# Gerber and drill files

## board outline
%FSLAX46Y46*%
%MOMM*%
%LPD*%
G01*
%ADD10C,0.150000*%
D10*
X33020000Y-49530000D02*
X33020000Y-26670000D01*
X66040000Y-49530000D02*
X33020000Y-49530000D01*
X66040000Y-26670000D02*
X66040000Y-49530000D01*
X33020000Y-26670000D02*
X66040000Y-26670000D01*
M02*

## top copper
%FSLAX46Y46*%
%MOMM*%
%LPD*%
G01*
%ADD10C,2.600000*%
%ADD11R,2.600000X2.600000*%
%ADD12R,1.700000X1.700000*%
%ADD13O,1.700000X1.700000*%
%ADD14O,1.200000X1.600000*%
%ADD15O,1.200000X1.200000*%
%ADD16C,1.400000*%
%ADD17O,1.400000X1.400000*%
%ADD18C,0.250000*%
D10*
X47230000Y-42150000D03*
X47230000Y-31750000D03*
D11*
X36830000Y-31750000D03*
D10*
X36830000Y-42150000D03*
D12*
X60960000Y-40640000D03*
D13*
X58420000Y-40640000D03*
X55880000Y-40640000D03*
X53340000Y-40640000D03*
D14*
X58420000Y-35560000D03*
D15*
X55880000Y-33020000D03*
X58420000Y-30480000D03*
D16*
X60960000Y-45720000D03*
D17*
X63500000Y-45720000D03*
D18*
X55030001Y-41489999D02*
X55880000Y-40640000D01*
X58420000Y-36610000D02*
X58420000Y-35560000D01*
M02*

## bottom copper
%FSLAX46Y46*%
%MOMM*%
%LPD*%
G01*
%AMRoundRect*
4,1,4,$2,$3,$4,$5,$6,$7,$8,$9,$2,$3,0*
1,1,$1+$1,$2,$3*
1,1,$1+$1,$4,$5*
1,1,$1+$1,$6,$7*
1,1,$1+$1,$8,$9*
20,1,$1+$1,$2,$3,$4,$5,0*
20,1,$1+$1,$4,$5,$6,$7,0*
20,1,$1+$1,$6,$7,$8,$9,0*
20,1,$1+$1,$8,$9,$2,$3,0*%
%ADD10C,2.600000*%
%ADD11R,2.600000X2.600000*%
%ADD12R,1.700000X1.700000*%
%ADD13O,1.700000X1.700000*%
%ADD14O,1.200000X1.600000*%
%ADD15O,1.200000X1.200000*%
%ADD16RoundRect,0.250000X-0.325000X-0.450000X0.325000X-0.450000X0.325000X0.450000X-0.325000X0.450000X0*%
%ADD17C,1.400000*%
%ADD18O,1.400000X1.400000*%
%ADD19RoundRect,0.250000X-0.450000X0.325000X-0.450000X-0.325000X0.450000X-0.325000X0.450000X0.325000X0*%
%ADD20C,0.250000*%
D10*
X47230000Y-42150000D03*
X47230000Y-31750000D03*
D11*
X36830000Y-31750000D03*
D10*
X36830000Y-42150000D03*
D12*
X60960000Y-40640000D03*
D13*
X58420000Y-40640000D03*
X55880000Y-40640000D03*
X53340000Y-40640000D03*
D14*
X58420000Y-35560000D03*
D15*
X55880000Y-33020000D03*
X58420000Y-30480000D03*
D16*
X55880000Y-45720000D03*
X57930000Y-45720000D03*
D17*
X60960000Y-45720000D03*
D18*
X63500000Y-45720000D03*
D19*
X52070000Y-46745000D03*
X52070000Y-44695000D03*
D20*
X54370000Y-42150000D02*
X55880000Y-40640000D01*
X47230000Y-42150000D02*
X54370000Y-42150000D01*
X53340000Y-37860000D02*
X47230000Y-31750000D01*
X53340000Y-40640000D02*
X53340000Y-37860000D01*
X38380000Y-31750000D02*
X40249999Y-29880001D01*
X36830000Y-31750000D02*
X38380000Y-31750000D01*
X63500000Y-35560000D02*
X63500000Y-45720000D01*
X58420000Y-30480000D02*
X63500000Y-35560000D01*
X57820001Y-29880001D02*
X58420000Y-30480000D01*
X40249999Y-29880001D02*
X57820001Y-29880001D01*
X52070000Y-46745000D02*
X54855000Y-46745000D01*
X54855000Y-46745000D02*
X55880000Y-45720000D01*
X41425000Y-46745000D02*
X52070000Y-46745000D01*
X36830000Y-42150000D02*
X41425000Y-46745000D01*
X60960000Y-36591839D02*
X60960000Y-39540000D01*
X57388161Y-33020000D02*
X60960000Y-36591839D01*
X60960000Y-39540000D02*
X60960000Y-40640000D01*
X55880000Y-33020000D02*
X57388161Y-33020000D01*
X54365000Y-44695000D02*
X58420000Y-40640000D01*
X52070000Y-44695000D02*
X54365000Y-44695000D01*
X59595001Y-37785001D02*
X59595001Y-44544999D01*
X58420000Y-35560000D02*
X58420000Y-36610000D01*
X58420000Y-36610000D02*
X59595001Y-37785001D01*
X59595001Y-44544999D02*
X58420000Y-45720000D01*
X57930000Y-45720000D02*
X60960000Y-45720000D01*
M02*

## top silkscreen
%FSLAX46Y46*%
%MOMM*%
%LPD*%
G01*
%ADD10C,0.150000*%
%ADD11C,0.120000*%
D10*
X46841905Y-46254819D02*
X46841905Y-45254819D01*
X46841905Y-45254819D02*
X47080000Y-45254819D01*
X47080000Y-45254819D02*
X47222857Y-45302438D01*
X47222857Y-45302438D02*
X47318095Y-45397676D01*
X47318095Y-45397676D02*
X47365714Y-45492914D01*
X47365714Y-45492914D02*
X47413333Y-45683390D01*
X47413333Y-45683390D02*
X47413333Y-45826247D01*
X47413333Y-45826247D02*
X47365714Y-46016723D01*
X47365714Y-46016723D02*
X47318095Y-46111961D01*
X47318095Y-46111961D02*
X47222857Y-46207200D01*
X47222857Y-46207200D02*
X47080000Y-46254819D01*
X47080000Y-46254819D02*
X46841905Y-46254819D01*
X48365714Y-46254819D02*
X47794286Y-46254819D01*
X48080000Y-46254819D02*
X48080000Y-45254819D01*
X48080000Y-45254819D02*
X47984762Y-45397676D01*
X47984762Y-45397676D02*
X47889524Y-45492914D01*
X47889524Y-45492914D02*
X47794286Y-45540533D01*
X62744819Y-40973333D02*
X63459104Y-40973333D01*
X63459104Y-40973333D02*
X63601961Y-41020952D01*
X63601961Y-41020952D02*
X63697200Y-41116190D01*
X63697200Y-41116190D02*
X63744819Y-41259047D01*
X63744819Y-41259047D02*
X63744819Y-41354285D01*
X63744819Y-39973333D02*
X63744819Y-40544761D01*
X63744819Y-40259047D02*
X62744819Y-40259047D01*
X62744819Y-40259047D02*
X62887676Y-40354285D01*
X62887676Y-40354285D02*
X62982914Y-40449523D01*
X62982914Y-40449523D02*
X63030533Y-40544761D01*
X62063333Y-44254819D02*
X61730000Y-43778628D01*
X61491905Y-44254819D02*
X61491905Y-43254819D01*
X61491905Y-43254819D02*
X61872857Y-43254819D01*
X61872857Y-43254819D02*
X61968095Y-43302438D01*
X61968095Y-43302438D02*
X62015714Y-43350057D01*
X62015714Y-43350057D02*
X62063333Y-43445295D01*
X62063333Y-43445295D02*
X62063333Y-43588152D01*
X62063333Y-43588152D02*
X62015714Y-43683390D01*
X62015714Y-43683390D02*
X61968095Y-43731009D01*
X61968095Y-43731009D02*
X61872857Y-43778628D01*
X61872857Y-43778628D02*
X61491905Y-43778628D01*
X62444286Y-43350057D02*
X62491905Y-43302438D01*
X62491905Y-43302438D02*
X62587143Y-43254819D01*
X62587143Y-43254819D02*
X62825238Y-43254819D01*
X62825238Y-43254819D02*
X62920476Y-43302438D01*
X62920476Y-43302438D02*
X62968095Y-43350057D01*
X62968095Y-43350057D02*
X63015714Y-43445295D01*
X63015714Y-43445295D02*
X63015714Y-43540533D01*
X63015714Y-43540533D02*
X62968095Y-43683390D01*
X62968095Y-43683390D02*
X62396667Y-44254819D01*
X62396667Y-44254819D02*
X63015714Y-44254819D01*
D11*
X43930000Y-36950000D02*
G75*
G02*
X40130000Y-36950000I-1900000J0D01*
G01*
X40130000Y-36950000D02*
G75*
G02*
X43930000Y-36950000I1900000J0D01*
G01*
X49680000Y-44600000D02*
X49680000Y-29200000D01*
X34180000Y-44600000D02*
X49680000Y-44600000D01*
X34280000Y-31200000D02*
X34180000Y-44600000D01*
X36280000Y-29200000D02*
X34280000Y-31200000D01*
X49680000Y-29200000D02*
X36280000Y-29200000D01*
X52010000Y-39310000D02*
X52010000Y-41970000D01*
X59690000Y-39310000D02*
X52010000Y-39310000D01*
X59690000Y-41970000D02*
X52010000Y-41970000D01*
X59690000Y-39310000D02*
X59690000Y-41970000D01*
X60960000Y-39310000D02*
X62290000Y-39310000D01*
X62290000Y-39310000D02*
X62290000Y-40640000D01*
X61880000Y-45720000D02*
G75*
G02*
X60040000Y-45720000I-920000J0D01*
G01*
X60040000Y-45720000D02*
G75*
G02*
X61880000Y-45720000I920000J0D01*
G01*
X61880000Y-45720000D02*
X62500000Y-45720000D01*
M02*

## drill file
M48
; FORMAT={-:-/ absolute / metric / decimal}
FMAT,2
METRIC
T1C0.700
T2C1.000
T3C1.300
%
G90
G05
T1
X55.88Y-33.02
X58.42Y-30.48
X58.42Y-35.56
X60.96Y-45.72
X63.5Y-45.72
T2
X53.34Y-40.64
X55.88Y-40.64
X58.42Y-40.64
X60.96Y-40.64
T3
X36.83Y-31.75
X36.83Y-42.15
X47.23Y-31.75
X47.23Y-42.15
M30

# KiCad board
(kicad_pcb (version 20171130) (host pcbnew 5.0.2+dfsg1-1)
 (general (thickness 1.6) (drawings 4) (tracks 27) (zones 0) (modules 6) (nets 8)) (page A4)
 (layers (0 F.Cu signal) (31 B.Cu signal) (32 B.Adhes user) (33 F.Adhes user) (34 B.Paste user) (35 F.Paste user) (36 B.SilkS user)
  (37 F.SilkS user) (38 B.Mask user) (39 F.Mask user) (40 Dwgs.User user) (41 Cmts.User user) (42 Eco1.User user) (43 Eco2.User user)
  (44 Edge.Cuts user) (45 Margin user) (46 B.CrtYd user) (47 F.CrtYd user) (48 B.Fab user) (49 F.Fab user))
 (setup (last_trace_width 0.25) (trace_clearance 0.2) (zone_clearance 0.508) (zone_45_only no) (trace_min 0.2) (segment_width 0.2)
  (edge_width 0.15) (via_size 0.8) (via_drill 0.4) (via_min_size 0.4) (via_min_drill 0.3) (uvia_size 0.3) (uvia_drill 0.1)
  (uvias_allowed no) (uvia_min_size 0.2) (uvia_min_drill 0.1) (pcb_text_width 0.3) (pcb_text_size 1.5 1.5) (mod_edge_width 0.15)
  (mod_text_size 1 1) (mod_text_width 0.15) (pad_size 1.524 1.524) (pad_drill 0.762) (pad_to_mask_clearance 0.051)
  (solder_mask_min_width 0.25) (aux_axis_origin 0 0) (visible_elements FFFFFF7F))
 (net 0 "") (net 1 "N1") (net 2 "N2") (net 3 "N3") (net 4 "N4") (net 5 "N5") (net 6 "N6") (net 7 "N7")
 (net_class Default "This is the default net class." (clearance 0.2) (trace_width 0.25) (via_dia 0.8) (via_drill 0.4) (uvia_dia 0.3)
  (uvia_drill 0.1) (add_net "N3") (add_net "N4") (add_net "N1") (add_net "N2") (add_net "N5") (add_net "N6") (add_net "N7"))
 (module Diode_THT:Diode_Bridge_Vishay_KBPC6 (layer F.Cu) (at 36.83 31.75)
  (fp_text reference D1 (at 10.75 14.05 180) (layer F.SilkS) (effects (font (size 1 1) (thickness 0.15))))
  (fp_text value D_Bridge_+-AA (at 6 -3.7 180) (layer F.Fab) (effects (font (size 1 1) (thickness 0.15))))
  (fp_circle (center 5.2 5.2) (end 5.2 7.1) (layer F.SilkS) (width 0.12))
  (fp_line (start 12.85 12.85) (end 12.85 -2.55) (layer F.SilkS) (width 0.12))
  (fp_line (start -2.65 12.85) (end 12.85 12.85) (layer F.SilkS) (width 0.12))
  (fp_line (start -2.55 -0.55) (end -2.65 12.85) (layer F.SilkS) (width 0.12))
  (fp_line (start -0.55 -2.55) (end -2.55 -0.55) (layer F.SilkS) (width 0.12))
  (fp_line (start 12.85 -2.55) (end -0.55 -2.55) (layer F.SilkS) (width 0.12))
  (pad 3 thru_hole circle (at 10.4 10.4) (size 2.6 2.6) (drill 1.3) (layers *.Cu *.Mask) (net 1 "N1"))
  (pad 4 thru_hole circle (at 10.4 0) (size 2.6 2.6) (drill 1.3) (layers *.Cu *.Mask) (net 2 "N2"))
  (pad 1 thru_hole rect (at 0 0) (size 2.6 2.6) (drill 1.3) (layers *.Cu *.Mask) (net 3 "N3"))
  (pad 2 thru_hole circle (at 0 10.4) (size 2.6 2.6) (drill 1.3) (layers *.Cu *.Mask) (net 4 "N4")))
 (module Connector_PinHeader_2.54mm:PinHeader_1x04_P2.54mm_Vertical (layer F.Cu) (at 60.96 40.64 270)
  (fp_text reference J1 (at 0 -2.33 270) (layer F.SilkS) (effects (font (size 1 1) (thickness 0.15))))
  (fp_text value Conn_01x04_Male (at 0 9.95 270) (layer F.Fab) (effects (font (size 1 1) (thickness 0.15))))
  (fp_line (start -1.33 8.95) (end 1.33 8.95) (layer F.SilkS) (width 0.12))
  (fp_line (start -1.33 1.27) (end -1.33 8.95) (layer F.SilkS) (width 0.12))
  (fp_line (start 1.33 1.27) (end 1.33 8.95) (layer F.SilkS) (width 0.12))
  (fp_line (start -1.33 1.27) (end 1.33 1.27) (layer F.SilkS) (width 0.12))
  (fp_line (start -1.33 0) (end -1.33 -1.33) (layer F.SilkS) (width 0.12))
  (fp_line (start -1.33 -1.33) (end 0 -1.33) (layer F.SilkS) (width 0.12))
  (pad 1 thru_hole rect (at 0 0 270) (size 1.7 1.7) (drill 1) (layers *.Cu *.Mask) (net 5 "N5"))
  (pad 2 thru_hole oval (at 0 2.54 270) (size 1.7 1.7) (drill 1) (layers *.Cu *.Mask) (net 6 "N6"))
  (pad 3 thru_hole oval (at 0 5.08 270) (size 1.7 1.7) (drill 1) (layers *.Cu *.Mask) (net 1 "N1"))
  (pad 4 thru_hole oval (at 0 7.62 270) (size 1.7 1.7) (drill 1) (layers *.Cu *.Mask) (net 2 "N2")))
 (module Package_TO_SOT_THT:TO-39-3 (layer B.Cu) (at 58.42 35.56 90)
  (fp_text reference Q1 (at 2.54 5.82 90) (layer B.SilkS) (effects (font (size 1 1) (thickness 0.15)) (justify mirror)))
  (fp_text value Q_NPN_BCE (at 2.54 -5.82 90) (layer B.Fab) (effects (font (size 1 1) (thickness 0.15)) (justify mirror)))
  (pad 1 thru_hole oval (at 0 0 90) (size 1.6 1.2) (drill 0.7) (layers *.Cu *.Mask) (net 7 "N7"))
  (pad 2 thru_hole oval (at 2.54 -2.54 90) (size 1.2 1.2) (drill 0.7) (layers *.Cu *.Mask) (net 5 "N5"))
  (pad 3 thru_hole oval (at 5.08 0 90) (size 1.2 1.2) (drill 0.7) (layers *.Cu *.Mask) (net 3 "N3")))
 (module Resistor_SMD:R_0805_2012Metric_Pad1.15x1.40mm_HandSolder (layer B.Cu) (at 56.905 45.72)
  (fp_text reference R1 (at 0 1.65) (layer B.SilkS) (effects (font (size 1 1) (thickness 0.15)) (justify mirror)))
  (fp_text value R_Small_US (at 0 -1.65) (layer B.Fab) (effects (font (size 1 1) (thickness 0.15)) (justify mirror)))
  (pad 1 smd roundrect (at -1.025 0) (size 1.15 1.4) (layers B.Cu B.Paste B.Mask) (roundrect_rratio 0.217391) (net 4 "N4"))
  (pad 2 smd roundrect (at 1.025 0) (size 1.15 1.4) (layers B.Cu B.Paste B.Mask) (roundrect_rratio 0.217391) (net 7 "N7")))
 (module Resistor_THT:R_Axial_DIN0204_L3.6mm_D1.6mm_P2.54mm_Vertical (layer F.Cu) (at 60.96 45.72)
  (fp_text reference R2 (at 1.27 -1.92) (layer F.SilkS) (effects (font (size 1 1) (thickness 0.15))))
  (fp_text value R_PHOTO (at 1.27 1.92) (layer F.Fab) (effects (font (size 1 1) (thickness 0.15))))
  (fp_circle (center 0 0) (end 0.92 0) (layer F.SilkS) (width 0.12))
  (fp_line (start 0.92 0) (end 1.54 0) (layer F.SilkS) (width 0.12))
  (pad 1 thru_hole circle (at 0 0) (size 1.4 1.4) (drill 0.7) (layers *.Cu *.Mask) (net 7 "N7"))
  (pad 2 thru_hole oval (at 2.54 0) (size 1.4 1.4) (drill 0.7) (layers *.Cu *.Mask) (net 3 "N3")))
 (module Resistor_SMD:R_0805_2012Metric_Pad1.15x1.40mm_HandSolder (layer B.Cu) (at 52.07 45.72 270)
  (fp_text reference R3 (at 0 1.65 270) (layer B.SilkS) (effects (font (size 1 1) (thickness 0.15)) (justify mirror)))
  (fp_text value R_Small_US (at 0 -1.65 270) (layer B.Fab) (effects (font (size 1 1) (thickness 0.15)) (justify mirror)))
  (pad 2 smd roundrect (at 1.025 0 270) (size 1.15 1.4) (layers B.Cu B.Paste B.Mask) (roundrect_rratio 0.217391) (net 4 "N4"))
  (pad 1 smd roundrect (at -1.025 0 270) (size 1.15 1.4) (layers B.Cu B.Paste B.Mask) (roundrect_rratio 0.217391) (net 6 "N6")))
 (gr_line (start 33.02 49.53) (end 33.02 26.67) (layer Edge.Cuts) (width 0.15))
 (gr_line (start 66.04 49.53) (end 33.02 49.53) (layer Edge.Cuts) (width 0.15))
 (gr_line (start 66.04 26.67) (end 66.04 49.53) (layer Edge.Cuts) (width 0.15))
 (gr_line (start 33.02 26.67) (end 66.04 26.67) (layer Edge.Cuts) (width 0.15))
 (segment (start 55.030001 41.489999) (end 55.88 40.64) (width 0.25) (layer F.Cu) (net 1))
 (segment (start 54.37 42.15) (end 55.88 40.64) (width 0.25) (layer B.Cu) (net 1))
 (segment (start 47.23 42.15) (end 54.37 42.15) (width 0.25) (layer B.Cu) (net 1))
 (segment (start 53.34 37.86) (end 47.23 31.75) (width 0.25) (layer B.Cu) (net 2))
 (segment (start 53.34 40.64) (end 53.34 37.86) (width 0.25) (layer B.Cu) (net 2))
 (segment (start 38.38 31.75) (end 40.249999 29.880001) (width 0.25) (layer B.Cu) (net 3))
 (segment (start 36.83 31.75) (end 38.38 31.75) (width 0.25) (layer B.Cu) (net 3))
 (segment (start 63.5 35.56) (end 63.5 45.72) (width 0.25) (layer B.Cu) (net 3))
 (segment (start 58.42 30.48) (end 63.5 35.56) (width 0.25) (layer B.Cu) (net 3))
 (segment (start 57.820001 29.880001) (end 58.42 30.48) (width 0.25) (layer B.Cu) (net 3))
 (segment (start 40.249999 29.880001) (end 57.820001 29.880001) (width 0.25) (layer B.Cu) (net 3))
 (segment (start 52.07 46.745) (end 54.855 46.745) (width 0.25) (layer B.Cu) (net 4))
 (segment (start 54.855 46.745) (end 55.88 45.72) (width 0.25) (layer B.Cu) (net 4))
 (segment (start 41.425 46.745) (end 52.07 46.745) (width 0.25) (layer B.Cu) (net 4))
 (segment (start 36.83 42.15) (end 41.425 46.745) (width 0.25) (layer B.Cu) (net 4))
 (segment (start 60.96 36.591839) (end 60.96 39.54) (width 0.25) (layer B.Cu) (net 5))
 (segment (start 57.388161 33.02) (end 60.96 36.591839) (width 0.25) (layer B.Cu) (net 5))
 (segment (start 60.96 39.54) (end 60.96 40.64) (width 0.25) (layer B.Cu) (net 5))
 (segment (start 55.88 33.02) (end 57.388161 33.02) (width 0.25) (layer B.Cu) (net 5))
 (segment (start 54.365 44.695) (end 58.42 40.64) (width 0.25) (layer B.Cu) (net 6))
 (segment (start 52.07 44.695) (end 54.365 44.695) (width 0.25) (layer B.Cu) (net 6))
 (segment (start 58.42 36.61) (end 58.42 35.56) (width 0.25) (layer F.Cu) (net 7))
 (segment (start 59.595001 37.785001) (end 59.595001 44.544999) (width 0.25) (layer B.Cu) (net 7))
 (segment (start 58.42 35.56) (end 58.42 36.61) (width 0.25) (layer B.Cu) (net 7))
 (segment (start 58.42 36.61) (end 59.595001 37.785001) (width 0.25) (layer B.Cu) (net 7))
 (segment (start 59.595001 44.544999) (end 58.42 45.72) (width 0.25) (layer B.Cu) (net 7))
 (segment (start 57.93 45.72) (end 60.96 45.72) (width 0.25) (layer B.Cu) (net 7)))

